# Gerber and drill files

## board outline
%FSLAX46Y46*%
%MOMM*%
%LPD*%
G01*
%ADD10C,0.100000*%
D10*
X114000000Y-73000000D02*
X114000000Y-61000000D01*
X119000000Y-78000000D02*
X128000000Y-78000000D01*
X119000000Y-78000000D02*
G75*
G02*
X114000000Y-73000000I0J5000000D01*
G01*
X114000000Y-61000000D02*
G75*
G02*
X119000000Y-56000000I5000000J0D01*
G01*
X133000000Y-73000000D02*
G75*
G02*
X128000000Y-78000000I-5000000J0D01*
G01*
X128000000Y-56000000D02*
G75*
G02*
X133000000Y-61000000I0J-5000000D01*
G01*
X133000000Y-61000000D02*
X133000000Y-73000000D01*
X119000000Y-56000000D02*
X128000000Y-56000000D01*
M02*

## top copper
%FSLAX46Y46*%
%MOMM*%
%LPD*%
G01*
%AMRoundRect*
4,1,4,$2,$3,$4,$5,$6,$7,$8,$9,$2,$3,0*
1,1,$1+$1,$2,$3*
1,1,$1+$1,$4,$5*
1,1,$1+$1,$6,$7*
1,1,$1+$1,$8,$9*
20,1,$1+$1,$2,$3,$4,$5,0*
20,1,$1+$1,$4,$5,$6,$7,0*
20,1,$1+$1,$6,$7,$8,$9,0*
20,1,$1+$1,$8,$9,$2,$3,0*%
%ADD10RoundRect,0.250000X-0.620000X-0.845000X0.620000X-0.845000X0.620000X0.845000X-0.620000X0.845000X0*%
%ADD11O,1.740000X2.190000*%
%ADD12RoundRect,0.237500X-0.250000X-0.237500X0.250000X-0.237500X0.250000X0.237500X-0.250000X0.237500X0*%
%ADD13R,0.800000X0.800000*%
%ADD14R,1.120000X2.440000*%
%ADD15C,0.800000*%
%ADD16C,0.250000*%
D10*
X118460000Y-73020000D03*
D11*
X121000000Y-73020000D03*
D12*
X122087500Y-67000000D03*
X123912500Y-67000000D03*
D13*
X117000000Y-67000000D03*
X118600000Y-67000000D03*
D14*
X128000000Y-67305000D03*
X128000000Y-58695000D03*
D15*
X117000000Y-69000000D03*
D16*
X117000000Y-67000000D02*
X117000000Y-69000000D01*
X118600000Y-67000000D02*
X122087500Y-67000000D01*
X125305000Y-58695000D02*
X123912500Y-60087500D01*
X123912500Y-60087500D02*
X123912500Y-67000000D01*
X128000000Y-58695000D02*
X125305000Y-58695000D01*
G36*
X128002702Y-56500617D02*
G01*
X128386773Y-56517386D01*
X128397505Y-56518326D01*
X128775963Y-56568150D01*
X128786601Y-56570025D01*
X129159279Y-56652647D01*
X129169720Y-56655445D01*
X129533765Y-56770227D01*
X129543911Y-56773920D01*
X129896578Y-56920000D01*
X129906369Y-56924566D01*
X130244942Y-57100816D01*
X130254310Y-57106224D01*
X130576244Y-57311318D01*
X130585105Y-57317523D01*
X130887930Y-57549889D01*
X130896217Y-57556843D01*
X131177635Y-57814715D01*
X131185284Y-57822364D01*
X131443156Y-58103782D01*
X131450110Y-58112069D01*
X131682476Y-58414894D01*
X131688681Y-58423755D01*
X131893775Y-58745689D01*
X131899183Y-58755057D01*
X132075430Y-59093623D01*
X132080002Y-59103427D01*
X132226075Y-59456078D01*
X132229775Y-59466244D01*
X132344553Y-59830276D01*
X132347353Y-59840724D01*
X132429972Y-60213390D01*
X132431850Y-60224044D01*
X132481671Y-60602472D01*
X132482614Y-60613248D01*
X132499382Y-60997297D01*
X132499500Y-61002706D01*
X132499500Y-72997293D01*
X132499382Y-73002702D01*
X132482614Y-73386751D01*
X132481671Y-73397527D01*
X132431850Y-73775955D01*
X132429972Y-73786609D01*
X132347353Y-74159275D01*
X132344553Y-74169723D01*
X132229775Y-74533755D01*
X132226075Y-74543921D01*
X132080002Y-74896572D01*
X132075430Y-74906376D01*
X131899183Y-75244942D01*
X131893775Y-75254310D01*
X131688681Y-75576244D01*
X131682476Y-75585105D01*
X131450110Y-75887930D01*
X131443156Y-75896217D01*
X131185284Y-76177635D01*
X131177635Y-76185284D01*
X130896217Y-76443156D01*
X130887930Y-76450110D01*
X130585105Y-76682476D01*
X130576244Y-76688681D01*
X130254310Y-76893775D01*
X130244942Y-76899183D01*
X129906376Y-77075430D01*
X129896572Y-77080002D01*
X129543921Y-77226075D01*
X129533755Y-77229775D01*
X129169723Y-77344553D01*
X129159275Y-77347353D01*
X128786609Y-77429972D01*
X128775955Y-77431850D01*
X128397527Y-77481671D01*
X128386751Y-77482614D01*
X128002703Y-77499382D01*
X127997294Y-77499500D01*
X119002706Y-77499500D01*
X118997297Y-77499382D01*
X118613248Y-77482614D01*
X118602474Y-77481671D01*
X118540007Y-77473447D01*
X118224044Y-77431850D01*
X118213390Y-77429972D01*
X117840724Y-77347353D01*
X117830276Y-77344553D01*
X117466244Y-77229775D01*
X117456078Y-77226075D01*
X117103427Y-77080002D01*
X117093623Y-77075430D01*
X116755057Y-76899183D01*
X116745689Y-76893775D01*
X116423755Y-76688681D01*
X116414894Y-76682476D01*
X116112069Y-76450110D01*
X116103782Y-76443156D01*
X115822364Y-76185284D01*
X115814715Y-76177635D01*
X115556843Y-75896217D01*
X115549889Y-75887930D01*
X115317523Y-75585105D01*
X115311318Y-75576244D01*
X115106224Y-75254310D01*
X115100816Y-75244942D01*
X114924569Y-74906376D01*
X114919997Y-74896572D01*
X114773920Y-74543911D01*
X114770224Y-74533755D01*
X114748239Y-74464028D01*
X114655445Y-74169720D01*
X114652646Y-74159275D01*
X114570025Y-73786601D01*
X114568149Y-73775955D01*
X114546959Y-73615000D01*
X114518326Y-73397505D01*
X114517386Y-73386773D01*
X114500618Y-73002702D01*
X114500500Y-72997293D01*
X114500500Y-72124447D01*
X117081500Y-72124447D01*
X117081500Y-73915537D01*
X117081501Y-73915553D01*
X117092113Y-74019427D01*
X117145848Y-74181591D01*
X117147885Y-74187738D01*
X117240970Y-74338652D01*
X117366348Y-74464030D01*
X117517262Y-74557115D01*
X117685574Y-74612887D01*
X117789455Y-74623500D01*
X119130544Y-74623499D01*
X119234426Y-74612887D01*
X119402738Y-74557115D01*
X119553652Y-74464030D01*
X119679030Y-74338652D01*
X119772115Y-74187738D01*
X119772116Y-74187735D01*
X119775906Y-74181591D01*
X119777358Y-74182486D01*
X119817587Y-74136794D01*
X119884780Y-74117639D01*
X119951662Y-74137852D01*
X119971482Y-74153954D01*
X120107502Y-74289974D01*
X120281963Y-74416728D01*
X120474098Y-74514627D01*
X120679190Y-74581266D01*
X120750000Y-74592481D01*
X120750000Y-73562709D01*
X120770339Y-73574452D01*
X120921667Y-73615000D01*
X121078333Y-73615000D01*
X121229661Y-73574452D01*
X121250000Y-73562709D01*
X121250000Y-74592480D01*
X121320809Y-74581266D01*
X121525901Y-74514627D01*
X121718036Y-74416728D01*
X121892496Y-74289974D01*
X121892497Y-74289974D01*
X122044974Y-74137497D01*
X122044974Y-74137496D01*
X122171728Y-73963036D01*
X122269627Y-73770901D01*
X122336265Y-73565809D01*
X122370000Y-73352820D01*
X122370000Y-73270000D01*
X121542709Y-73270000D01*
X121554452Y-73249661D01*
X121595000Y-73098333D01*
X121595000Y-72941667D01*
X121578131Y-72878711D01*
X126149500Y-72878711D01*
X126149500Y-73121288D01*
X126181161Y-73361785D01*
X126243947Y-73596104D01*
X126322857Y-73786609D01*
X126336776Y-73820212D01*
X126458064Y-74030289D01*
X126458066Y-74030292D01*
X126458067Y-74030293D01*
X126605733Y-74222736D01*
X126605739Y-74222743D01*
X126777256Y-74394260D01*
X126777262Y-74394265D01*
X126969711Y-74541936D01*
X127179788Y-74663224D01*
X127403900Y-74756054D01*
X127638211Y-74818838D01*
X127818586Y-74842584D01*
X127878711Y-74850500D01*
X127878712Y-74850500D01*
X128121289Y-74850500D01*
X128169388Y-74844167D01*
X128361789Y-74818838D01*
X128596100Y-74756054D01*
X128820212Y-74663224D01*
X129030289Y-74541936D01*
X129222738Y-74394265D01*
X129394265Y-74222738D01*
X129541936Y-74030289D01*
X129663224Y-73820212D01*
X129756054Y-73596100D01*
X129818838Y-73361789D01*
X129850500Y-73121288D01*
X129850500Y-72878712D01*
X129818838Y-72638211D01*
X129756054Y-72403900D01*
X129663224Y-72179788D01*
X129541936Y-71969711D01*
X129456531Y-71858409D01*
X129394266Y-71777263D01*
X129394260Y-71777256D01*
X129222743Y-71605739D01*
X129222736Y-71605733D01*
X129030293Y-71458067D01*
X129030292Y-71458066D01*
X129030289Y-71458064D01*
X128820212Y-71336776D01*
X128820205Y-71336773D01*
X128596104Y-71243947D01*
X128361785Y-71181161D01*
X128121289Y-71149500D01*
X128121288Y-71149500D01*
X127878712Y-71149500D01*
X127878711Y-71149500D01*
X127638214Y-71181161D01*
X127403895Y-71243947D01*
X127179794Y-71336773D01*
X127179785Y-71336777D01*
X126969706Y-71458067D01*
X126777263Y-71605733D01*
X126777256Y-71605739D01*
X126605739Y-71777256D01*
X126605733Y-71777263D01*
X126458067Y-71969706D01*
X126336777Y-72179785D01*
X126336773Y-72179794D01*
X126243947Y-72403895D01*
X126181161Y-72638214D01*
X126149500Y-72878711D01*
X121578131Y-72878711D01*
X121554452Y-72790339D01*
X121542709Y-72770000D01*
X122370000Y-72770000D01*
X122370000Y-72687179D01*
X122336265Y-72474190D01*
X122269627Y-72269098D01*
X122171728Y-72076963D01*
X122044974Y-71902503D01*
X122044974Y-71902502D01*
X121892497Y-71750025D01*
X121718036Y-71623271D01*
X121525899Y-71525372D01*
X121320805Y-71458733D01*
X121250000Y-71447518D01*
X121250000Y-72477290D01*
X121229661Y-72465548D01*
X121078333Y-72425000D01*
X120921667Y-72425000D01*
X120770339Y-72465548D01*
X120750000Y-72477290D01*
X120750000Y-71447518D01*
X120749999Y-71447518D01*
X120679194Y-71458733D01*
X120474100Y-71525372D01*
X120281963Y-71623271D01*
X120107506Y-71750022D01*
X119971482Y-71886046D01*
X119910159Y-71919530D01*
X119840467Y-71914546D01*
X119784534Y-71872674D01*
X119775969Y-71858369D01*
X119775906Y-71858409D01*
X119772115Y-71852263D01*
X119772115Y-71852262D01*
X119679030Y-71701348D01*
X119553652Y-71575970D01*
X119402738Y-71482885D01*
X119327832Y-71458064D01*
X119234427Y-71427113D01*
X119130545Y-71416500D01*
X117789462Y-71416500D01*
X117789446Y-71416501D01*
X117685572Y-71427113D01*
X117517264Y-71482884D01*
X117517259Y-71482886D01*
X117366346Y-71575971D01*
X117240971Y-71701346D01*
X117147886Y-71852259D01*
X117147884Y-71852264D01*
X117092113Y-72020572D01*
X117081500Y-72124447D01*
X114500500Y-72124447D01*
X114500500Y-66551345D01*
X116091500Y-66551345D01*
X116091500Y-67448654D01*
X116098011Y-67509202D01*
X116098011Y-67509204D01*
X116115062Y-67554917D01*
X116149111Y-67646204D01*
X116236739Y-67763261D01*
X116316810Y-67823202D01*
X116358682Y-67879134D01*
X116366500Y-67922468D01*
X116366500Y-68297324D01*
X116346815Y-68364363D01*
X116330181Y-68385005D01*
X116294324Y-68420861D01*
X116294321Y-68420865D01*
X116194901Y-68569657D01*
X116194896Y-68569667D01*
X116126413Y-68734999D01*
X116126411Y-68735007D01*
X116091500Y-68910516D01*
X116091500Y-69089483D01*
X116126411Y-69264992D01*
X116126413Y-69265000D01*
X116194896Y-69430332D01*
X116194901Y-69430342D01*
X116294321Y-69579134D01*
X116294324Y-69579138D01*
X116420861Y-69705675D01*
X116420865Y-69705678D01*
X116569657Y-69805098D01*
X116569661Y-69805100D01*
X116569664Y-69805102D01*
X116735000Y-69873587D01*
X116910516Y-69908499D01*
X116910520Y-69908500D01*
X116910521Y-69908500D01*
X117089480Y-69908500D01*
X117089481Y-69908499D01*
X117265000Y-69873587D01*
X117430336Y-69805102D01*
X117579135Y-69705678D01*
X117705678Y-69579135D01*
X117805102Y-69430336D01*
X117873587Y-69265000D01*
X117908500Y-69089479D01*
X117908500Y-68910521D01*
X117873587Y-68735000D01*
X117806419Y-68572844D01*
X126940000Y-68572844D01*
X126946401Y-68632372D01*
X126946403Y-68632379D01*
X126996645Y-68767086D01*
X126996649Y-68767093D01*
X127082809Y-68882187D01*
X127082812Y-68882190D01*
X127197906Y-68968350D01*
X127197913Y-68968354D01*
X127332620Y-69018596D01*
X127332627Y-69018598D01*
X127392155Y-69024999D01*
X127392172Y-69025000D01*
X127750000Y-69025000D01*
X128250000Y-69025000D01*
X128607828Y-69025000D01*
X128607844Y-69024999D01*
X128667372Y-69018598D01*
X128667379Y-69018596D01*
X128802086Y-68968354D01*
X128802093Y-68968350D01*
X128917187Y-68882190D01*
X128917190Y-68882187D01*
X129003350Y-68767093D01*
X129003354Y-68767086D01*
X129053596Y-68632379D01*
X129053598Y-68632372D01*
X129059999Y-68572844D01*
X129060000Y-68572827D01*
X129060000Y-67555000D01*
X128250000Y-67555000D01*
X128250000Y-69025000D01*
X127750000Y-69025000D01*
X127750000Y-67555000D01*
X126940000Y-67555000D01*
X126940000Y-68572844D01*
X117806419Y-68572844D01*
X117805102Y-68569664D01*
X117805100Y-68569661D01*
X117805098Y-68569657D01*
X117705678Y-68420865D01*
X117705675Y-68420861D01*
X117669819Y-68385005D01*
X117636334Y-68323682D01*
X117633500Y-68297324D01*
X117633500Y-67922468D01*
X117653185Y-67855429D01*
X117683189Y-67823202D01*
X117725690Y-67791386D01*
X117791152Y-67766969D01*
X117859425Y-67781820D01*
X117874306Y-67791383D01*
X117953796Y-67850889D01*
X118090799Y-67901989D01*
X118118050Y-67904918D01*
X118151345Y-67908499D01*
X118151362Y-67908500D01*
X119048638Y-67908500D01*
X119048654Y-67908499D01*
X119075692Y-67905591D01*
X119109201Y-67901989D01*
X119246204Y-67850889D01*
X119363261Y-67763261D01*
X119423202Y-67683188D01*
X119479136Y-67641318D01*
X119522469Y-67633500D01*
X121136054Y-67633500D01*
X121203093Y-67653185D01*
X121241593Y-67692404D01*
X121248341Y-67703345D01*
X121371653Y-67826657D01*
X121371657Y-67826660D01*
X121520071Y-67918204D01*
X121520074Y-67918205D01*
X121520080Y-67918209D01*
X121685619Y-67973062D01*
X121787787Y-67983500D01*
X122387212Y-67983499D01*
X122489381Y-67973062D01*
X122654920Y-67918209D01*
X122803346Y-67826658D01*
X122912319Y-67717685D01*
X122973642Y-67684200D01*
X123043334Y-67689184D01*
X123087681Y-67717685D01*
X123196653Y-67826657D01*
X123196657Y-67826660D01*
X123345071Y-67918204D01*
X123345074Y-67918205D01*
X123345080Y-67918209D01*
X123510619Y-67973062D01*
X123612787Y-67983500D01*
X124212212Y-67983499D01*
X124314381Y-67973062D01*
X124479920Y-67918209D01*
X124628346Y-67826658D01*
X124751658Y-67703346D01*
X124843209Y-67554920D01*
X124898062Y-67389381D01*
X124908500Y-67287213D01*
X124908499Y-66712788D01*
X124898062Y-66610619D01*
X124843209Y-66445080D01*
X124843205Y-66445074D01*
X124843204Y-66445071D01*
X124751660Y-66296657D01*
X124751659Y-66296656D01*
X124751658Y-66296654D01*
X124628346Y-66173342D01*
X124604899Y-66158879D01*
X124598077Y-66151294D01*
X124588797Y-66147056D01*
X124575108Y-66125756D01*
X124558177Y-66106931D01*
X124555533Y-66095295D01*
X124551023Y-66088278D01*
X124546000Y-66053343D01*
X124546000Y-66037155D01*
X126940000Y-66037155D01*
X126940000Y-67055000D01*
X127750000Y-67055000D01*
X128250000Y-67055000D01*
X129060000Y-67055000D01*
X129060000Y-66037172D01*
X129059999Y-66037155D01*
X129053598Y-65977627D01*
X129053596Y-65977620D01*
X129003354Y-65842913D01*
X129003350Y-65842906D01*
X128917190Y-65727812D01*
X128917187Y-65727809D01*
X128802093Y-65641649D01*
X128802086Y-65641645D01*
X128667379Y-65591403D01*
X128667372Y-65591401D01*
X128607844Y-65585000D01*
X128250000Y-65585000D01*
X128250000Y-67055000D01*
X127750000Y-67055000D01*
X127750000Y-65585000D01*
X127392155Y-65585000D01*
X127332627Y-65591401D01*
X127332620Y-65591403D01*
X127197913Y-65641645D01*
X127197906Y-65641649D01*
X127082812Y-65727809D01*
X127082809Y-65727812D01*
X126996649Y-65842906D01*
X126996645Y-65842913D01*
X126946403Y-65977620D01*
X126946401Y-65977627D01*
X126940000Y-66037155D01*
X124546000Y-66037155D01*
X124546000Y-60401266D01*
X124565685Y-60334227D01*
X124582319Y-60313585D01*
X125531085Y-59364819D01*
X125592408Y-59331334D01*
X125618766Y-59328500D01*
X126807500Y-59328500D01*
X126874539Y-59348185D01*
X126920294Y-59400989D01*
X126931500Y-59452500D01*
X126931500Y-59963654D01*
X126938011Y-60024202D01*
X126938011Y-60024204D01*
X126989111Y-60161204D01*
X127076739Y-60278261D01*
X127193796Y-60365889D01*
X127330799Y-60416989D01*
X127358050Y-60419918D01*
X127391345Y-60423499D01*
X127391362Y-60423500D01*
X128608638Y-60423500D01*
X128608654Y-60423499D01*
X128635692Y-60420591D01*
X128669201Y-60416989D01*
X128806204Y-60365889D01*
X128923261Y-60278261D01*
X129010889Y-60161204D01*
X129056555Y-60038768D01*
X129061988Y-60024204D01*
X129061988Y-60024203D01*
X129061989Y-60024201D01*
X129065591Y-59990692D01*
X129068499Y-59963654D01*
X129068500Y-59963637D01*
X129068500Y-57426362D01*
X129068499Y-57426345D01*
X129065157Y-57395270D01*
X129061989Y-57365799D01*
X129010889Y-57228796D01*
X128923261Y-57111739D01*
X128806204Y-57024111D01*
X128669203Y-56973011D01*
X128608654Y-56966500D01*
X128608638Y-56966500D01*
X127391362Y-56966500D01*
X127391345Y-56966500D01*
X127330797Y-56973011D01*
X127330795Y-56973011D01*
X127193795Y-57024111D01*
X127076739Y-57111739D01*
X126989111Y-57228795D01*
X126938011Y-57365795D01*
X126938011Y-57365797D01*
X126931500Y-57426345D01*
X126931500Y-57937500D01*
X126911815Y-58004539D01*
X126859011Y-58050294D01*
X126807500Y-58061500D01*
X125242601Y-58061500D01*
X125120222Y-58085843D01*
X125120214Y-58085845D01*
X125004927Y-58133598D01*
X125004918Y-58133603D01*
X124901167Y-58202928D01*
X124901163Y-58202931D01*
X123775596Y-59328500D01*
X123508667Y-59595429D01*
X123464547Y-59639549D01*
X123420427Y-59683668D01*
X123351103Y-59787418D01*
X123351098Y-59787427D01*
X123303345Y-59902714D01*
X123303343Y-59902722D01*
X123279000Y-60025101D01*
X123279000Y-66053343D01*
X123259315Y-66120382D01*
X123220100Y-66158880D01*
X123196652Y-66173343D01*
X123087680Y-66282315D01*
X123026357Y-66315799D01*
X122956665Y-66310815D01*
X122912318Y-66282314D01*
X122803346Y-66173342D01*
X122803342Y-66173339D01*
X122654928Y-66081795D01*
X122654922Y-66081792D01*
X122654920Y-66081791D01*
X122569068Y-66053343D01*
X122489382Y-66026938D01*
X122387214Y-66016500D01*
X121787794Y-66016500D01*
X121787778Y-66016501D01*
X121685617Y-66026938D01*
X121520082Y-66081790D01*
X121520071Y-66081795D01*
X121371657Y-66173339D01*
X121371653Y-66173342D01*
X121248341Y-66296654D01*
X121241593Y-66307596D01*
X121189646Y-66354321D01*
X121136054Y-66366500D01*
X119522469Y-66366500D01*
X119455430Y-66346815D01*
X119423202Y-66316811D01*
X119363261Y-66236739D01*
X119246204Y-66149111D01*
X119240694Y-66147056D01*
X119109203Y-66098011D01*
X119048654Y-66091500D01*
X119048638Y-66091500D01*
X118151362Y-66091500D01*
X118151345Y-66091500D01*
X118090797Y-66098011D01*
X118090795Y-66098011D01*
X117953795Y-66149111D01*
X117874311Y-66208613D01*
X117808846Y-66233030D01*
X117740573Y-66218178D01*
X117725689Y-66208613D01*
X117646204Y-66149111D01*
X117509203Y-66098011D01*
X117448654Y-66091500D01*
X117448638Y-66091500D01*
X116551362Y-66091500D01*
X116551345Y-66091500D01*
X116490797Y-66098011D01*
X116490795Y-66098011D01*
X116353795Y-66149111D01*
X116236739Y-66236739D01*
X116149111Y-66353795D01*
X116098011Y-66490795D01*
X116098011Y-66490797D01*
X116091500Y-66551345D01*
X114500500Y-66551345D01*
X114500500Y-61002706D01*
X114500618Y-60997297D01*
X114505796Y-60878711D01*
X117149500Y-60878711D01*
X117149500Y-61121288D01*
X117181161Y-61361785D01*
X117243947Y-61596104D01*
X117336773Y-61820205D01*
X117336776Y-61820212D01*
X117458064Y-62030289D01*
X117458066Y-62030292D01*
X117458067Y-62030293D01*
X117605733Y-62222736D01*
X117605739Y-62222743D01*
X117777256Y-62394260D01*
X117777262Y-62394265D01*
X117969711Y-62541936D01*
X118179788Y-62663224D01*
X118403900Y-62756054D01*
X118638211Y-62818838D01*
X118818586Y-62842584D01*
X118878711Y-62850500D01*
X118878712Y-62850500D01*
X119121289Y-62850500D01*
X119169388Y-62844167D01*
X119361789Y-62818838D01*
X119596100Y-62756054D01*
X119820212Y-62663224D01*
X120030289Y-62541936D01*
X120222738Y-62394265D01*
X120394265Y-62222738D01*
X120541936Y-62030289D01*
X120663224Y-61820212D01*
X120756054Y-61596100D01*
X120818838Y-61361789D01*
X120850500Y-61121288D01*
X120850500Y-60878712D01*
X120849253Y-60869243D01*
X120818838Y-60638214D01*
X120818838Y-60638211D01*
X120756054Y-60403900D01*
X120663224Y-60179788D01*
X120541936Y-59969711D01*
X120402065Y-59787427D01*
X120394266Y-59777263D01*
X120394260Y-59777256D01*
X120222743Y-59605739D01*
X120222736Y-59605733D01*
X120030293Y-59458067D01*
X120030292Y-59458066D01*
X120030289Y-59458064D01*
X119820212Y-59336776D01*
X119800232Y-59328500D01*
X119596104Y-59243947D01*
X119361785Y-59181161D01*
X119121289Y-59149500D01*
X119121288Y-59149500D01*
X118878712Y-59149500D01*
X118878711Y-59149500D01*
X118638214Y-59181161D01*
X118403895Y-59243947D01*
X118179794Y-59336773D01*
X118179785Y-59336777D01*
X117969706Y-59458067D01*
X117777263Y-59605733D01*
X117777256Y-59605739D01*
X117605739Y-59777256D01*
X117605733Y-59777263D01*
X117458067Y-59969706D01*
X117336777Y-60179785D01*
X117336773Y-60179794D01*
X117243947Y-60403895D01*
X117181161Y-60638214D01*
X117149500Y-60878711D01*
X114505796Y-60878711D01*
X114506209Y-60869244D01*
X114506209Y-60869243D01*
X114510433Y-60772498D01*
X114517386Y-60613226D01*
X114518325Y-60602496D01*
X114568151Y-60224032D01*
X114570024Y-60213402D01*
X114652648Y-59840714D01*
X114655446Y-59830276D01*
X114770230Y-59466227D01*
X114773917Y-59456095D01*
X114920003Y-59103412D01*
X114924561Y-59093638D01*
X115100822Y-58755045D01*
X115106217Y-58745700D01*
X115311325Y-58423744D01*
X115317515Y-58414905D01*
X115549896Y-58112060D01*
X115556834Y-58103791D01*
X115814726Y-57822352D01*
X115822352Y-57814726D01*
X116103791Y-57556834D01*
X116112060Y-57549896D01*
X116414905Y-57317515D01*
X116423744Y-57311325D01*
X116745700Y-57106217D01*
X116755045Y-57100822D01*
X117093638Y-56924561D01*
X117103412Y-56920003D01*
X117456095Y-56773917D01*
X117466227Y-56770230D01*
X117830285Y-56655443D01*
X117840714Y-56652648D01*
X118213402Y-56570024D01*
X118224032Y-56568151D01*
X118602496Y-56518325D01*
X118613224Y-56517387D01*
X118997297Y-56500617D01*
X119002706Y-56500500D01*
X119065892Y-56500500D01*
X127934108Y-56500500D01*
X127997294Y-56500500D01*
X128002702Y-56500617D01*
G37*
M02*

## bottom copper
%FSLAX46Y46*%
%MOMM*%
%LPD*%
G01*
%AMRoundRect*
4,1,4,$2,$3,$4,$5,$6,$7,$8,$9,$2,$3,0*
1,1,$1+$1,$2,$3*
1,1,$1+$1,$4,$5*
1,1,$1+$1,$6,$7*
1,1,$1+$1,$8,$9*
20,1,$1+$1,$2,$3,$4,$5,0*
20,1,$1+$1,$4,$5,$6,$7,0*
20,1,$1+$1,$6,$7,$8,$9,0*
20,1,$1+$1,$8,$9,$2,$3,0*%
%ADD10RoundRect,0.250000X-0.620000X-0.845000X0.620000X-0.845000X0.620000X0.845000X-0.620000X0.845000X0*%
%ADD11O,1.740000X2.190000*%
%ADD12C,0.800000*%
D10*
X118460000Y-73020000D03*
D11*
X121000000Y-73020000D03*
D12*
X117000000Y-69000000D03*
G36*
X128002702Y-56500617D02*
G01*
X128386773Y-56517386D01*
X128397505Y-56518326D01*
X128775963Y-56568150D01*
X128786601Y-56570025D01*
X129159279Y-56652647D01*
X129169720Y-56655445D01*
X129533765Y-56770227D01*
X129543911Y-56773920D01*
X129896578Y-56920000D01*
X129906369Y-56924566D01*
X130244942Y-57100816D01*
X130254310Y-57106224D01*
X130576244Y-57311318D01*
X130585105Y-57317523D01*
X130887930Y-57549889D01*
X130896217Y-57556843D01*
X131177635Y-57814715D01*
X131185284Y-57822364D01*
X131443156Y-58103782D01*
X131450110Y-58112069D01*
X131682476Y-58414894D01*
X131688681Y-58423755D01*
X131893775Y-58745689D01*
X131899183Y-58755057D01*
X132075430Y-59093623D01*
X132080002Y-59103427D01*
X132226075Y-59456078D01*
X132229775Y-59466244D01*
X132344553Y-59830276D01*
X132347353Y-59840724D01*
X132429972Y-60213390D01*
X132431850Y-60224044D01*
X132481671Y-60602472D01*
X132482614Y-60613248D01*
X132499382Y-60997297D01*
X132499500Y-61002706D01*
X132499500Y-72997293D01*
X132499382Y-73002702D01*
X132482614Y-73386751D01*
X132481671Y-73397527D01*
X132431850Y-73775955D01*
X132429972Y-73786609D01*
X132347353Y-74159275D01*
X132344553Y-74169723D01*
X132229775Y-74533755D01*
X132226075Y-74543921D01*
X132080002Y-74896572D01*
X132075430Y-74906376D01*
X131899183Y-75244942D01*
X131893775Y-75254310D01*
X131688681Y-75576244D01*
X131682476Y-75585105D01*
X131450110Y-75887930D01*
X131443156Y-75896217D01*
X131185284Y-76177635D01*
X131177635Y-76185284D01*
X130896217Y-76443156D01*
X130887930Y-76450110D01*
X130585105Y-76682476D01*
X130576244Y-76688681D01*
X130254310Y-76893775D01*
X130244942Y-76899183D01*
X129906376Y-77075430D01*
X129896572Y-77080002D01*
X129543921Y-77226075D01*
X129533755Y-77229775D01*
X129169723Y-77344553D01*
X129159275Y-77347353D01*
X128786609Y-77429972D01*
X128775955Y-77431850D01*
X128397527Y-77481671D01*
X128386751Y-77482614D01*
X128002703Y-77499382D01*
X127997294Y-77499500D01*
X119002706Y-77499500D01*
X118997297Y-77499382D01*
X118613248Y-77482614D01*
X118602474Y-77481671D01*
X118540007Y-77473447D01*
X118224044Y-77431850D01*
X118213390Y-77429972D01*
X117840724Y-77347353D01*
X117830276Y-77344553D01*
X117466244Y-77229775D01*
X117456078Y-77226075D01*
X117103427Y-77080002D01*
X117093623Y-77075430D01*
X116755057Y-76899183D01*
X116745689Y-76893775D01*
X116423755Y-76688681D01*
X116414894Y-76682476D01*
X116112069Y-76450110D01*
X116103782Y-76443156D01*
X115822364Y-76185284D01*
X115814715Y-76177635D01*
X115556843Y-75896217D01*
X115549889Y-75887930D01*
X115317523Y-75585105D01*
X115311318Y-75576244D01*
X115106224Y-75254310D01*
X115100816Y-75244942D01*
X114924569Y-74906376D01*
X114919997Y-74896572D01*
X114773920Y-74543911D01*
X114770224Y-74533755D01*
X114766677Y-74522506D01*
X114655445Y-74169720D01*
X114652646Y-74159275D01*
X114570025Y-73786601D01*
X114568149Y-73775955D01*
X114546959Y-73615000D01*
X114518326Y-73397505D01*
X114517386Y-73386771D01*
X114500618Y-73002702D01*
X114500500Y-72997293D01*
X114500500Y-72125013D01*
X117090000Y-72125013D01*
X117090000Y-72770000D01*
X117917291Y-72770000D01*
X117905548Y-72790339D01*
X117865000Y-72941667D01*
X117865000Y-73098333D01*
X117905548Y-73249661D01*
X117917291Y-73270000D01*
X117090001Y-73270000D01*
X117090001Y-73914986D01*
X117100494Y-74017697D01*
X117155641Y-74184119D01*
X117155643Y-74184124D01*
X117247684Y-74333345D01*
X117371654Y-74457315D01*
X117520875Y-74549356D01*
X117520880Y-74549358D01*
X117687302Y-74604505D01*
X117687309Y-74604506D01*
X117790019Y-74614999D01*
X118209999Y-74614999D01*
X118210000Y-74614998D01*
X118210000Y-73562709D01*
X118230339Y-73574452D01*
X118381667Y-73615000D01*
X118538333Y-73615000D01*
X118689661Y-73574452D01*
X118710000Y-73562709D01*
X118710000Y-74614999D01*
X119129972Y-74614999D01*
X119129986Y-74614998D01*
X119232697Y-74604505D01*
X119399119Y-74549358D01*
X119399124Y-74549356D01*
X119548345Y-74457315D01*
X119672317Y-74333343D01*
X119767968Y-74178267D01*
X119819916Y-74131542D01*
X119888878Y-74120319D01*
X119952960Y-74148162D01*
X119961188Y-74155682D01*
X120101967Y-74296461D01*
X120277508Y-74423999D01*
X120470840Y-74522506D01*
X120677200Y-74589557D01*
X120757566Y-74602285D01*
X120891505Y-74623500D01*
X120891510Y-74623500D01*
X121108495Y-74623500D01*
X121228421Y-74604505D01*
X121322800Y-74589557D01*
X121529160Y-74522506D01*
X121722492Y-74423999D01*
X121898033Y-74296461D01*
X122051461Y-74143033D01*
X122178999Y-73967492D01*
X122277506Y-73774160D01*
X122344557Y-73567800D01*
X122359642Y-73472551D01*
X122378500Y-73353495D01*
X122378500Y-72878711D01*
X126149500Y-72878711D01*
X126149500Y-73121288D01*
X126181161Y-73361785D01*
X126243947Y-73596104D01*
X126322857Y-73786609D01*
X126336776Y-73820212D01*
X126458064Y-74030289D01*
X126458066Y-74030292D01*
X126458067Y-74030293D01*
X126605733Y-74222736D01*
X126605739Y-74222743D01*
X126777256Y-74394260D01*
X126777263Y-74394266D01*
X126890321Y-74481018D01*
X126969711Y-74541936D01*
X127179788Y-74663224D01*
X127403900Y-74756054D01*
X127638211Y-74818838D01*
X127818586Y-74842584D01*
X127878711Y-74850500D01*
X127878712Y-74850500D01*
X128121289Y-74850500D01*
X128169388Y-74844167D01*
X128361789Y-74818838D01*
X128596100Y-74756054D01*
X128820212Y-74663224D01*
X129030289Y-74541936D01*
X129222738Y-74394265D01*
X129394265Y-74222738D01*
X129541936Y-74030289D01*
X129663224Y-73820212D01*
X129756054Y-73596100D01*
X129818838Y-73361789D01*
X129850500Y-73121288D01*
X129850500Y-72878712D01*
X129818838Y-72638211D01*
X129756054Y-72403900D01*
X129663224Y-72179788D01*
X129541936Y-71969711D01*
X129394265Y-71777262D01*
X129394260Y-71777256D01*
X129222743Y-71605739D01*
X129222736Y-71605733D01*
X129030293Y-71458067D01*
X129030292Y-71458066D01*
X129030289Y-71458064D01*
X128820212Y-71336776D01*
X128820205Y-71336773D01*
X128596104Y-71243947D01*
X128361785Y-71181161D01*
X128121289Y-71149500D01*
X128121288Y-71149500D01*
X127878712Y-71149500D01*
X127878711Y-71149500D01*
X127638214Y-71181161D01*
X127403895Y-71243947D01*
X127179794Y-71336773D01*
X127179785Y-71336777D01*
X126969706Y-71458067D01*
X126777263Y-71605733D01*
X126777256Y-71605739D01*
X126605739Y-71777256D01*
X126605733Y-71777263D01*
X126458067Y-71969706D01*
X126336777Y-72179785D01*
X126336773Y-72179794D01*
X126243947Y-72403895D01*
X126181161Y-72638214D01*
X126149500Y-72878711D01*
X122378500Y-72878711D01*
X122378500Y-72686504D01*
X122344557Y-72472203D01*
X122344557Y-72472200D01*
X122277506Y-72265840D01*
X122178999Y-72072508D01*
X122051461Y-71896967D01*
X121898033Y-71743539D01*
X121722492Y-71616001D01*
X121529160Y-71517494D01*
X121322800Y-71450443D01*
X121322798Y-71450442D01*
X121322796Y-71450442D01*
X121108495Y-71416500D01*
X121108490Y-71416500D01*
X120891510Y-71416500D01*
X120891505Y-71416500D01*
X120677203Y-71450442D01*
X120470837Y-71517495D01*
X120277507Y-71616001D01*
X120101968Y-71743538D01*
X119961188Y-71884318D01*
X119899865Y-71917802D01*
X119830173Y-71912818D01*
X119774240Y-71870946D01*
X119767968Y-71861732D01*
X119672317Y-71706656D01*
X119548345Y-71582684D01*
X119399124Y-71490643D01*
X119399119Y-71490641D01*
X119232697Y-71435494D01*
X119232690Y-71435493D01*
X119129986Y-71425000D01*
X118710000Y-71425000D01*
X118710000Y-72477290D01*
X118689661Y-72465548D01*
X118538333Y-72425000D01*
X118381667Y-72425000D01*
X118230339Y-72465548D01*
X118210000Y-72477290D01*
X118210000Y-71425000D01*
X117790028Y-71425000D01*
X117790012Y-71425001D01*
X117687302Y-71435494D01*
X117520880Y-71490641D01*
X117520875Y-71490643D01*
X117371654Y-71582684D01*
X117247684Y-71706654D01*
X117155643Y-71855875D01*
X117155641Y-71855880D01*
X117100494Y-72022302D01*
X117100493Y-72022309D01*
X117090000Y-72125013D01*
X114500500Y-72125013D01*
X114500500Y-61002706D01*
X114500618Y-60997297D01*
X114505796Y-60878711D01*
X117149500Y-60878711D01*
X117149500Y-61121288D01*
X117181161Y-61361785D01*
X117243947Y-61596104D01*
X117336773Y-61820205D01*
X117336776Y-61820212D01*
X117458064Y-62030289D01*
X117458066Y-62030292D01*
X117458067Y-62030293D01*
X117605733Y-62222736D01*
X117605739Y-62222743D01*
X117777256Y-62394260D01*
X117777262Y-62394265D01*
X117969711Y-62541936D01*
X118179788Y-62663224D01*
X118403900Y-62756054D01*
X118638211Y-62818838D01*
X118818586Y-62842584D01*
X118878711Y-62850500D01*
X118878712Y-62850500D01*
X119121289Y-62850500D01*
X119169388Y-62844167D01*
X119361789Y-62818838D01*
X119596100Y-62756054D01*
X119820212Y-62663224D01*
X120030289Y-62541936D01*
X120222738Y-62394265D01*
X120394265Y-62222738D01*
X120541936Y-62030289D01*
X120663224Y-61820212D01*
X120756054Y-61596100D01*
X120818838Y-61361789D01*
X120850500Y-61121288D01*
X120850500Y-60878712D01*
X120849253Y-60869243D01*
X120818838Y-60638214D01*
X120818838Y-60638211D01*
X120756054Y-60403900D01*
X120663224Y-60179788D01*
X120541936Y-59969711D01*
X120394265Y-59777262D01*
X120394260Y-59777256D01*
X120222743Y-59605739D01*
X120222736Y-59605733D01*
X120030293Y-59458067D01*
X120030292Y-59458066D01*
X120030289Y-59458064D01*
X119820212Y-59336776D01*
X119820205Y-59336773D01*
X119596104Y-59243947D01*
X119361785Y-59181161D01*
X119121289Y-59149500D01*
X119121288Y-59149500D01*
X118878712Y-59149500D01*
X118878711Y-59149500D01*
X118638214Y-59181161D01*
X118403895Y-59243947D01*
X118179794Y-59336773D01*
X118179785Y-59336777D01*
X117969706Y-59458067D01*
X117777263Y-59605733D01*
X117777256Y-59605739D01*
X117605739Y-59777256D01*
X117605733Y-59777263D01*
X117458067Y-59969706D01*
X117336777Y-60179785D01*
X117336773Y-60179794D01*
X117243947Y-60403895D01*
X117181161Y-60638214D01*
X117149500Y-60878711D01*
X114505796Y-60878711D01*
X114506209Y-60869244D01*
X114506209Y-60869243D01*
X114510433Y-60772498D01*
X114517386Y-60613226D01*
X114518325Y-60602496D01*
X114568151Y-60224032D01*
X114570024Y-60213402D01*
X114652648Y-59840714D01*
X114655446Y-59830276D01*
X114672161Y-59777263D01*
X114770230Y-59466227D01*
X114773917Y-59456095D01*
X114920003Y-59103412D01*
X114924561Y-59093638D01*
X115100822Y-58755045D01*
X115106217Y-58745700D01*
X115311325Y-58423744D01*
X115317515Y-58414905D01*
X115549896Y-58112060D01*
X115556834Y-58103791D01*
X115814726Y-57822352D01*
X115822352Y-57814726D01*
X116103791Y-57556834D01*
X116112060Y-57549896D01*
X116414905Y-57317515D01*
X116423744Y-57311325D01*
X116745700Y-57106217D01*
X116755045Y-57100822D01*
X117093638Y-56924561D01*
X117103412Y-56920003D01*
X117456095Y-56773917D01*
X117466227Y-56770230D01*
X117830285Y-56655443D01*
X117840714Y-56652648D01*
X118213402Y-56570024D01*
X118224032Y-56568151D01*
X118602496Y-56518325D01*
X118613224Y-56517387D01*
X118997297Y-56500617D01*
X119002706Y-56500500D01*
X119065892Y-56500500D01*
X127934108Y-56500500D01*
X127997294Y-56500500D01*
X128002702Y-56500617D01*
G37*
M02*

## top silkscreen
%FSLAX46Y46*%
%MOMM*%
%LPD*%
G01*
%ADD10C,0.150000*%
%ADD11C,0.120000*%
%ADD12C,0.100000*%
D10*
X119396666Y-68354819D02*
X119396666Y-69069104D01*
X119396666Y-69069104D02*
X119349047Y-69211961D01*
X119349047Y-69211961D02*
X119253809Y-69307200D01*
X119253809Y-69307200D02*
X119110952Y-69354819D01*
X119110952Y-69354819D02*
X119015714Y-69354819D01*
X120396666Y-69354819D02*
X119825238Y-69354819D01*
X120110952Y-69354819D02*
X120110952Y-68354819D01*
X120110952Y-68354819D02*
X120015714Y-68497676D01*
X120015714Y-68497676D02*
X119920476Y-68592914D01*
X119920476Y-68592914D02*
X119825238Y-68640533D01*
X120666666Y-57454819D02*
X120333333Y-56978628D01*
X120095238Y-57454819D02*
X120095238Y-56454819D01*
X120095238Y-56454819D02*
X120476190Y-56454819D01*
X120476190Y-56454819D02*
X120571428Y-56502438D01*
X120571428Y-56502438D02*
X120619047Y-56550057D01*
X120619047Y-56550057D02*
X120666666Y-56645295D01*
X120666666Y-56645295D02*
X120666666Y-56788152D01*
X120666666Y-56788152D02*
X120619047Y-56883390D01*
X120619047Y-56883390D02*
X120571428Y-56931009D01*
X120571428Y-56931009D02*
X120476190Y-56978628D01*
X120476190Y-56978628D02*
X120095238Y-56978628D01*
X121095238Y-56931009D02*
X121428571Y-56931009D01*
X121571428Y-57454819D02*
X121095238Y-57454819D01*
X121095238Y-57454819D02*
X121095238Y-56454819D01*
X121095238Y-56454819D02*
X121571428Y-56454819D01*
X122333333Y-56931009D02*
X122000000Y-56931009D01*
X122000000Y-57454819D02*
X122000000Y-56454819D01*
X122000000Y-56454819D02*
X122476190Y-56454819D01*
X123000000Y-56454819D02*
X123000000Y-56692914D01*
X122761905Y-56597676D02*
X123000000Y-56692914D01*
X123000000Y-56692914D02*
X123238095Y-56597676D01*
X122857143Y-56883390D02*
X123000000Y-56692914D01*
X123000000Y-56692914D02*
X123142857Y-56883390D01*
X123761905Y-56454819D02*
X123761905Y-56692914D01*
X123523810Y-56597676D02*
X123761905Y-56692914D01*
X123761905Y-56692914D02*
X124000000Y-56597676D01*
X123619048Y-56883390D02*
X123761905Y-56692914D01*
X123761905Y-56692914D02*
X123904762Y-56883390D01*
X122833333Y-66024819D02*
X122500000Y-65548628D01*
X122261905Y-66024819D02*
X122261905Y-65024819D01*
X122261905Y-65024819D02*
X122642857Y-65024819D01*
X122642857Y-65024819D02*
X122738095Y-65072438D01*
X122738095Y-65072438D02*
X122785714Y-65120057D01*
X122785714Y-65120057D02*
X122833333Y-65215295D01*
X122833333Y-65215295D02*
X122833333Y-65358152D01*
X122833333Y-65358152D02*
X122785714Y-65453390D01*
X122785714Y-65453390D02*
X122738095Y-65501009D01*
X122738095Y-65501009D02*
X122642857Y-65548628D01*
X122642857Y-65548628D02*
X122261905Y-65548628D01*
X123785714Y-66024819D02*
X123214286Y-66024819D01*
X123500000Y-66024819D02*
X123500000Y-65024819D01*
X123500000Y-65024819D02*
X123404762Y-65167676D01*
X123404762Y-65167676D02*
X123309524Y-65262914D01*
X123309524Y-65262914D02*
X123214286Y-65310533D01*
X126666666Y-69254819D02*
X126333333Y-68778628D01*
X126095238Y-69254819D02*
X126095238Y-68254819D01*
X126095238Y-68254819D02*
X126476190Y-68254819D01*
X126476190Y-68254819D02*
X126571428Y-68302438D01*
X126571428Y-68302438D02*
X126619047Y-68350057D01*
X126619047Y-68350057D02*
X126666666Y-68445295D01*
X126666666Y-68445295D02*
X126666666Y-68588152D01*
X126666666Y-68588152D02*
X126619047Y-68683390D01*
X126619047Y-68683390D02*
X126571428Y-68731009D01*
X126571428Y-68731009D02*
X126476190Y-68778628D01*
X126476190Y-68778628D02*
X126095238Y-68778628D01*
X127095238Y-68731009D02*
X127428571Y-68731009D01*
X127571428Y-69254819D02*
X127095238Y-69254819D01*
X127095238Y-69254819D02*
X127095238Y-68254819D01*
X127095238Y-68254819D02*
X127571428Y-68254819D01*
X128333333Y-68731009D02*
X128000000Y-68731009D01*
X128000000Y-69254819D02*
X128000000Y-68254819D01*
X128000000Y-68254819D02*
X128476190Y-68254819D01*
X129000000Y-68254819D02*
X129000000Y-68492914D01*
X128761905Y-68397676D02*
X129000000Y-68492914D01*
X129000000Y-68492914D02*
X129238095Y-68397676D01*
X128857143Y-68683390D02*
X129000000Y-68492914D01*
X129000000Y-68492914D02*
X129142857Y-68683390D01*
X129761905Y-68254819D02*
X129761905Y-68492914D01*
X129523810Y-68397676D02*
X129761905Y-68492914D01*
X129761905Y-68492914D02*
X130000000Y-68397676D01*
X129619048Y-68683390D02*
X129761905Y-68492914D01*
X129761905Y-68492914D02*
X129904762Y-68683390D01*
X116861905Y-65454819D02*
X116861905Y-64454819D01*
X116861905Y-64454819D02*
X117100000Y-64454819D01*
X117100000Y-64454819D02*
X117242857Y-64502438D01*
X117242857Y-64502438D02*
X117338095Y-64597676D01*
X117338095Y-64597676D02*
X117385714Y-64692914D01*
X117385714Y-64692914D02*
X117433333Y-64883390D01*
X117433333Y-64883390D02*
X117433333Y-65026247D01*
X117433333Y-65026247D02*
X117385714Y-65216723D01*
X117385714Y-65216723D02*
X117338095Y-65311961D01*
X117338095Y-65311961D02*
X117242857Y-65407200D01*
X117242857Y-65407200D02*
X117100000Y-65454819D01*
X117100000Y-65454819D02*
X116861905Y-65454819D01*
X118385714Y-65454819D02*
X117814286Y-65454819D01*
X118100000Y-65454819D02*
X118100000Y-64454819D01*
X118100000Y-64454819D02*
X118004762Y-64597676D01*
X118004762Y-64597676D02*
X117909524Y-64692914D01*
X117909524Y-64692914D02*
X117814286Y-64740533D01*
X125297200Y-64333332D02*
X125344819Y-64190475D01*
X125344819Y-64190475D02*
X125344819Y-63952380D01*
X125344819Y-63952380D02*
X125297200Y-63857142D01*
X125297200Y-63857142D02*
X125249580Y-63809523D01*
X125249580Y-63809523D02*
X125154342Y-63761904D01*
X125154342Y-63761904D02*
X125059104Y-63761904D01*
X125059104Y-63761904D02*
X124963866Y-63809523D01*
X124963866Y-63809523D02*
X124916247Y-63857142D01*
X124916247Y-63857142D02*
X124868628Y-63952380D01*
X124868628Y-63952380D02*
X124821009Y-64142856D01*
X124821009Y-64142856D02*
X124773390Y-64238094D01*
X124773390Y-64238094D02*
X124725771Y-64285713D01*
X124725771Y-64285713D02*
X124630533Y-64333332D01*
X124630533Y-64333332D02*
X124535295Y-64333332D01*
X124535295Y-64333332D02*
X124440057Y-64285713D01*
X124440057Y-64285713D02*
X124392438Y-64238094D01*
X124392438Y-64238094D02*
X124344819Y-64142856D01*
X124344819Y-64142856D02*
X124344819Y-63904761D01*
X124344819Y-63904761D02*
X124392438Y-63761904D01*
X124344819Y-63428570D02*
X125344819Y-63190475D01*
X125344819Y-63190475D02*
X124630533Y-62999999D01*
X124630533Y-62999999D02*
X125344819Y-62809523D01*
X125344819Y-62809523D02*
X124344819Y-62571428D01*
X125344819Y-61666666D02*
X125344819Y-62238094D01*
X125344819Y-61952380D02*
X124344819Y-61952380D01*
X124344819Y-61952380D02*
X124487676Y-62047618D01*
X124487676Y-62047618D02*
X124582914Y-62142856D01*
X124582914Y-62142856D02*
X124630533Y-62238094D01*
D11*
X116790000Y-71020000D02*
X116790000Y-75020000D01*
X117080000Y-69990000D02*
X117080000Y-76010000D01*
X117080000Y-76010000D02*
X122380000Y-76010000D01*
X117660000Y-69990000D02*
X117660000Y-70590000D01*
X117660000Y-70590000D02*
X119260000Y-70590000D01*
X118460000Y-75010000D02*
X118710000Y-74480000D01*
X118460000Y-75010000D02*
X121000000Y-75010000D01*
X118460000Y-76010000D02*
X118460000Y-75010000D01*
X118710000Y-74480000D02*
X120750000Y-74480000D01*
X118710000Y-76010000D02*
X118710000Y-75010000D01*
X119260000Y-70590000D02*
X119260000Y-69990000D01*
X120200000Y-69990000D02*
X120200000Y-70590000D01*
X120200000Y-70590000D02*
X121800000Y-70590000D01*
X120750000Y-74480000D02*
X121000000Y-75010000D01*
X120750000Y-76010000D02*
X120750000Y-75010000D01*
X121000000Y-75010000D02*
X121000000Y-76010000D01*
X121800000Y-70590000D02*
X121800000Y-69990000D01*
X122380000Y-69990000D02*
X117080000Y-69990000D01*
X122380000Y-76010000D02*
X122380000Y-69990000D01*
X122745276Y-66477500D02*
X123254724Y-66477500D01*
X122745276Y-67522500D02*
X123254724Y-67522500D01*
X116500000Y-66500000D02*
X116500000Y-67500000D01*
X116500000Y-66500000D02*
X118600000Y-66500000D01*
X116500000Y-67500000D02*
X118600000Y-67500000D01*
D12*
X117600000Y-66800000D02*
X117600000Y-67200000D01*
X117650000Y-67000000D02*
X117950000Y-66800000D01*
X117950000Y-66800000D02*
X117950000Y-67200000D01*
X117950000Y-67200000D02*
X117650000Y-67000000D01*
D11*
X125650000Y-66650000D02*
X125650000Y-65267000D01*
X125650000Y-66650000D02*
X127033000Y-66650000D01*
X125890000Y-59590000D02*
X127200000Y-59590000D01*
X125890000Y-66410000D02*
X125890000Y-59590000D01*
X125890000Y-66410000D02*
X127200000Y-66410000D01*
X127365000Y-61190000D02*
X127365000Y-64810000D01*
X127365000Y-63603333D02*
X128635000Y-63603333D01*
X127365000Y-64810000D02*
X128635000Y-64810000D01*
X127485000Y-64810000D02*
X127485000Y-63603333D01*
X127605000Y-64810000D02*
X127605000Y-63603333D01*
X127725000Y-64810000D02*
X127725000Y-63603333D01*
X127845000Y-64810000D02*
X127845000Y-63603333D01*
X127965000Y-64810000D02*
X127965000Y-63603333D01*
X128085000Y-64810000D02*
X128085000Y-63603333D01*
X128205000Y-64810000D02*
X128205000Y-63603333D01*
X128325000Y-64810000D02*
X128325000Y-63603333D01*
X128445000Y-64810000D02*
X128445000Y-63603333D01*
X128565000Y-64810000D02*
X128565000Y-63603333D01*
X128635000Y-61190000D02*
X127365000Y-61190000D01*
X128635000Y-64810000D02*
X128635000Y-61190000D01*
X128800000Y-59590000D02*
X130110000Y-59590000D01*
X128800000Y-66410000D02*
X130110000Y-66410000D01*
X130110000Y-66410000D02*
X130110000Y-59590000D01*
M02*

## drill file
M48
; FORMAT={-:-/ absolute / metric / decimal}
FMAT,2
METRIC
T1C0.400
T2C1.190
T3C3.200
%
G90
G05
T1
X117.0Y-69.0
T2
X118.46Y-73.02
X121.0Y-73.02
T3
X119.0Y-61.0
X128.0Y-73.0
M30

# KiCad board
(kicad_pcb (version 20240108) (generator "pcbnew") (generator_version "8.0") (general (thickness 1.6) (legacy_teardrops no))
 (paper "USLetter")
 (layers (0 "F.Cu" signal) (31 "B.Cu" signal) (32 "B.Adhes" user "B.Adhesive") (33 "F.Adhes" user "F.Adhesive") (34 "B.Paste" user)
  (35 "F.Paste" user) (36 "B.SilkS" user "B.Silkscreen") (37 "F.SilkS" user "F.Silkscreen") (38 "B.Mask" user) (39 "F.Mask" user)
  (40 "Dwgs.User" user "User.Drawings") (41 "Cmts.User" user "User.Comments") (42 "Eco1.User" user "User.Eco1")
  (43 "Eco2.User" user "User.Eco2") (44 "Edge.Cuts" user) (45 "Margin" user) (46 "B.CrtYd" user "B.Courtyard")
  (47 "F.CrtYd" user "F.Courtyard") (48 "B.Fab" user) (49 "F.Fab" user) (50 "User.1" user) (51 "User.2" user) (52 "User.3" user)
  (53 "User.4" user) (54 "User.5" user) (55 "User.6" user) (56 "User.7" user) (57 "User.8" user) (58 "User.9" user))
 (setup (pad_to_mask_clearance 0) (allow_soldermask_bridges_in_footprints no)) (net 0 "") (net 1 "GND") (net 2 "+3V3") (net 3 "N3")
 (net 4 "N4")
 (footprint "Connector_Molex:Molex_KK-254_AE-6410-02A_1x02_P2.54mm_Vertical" (layer "F.Cu") (at 118.46 73.02)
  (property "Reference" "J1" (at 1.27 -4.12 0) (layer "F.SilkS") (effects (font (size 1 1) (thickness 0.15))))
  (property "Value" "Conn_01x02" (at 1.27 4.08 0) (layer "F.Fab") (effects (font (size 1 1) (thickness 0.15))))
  (fp_line (start -1.67 -2) (end -1.67 2) (stroke (width 0.12) (type solid)) (layer "F.SilkS"))
  (fp_line (start -1.38 -3.03) (end -1.38 2.99) (stroke (width 0.12) (type solid)) (layer "F.SilkS"))
  (fp_line (start -1.38 2.99) (end 3.92 2.99) (stroke (width 0.12) (type solid)) (layer "F.SilkS"))
  (fp_line (start -0.8 -3.03) (end -0.8 -2.43) (stroke (width 0.12) (type solid)) (layer "F.SilkS"))
  (fp_line (start -0.8 -2.43) (end 0.8 -2.43) (stroke (width 0.12) (type solid)) (layer "F.SilkS"))
  (fp_line (start 0 1.99) (end 0.25 1.46) (stroke (width 0.12) (type solid)) (layer "F.SilkS"))
  (fp_line (start 0 1.99) (end 2.54 1.99) (stroke (width 0.12) (type solid)) (layer "F.SilkS"))
  (fp_line (start 0 2.99) (end 0 1.99) (stroke (width 0.12) (type solid)) (layer "F.SilkS"))
  (fp_line (start 0.25 1.46) (end 2.29 1.46) (stroke (width 0.12) (type solid)) (layer "F.SilkS"))
  (fp_line (start 0.25 2.99) (end 0.25 1.99) (stroke (width 0.12) (type solid)) (layer "F.SilkS"))
  (fp_line (start 0.8 -2.43) (end 0.8 -3.03) (stroke (width 0.12) (type solid)) (layer "F.SilkS"))
  (fp_line (start 1.74 -3.03) (end 1.74 -2.43) (stroke (width 0.12) (type solid)) (layer "F.SilkS"))
  (fp_line (start 1.74 -2.43) (end 3.34 -2.43) (stroke (width 0.12) (type solid)) (layer "F.SilkS"))
  (fp_line (start 2.29 1.46) (end 2.54 1.99) (stroke (width 0.12) (type solid)) (layer "F.SilkS"))
  (fp_line (start 2.29 2.99) (end 2.29 1.99) (stroke (width 0.12) (type solid)) (layer "F.SilkS"))
  (fp_line (start 2.54 1.99) (end 2.54 2.99) (stroke (width 0.12) (type solid)) (layer "F.SilkS"))
  (fp_line (start 3.34 -2.43) (end 3.34 -3.03) (stroke (width 0.12) (type solid)) (layer "F.SilkS"))
  (fp_line (start 3.92 -3.03) (end -1.38 -3.03) (stroke (width 0.12) (type solid)) (layer "F.SilkS"))
  (fp_line (start 3.92 2.99) (end 3.92 -3.03) (stroke (width 0.12) (type solid)) (layer "F.SilkS"))
  (pad "1" thru_hole roundrect (at 0 0) (size 1.74 2.19) (drill 1.19) (layers "*.Cu" "*.Mask") (remove_unused_layers no)
   (roundrect_rratio 0.143678) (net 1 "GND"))
  (pad "2" thru_hole oval (at 2.54 0) (size 1.74 2.19) (drill 1.19) (layers "*.Cu" "*.Mask") (remove_unused_layers no) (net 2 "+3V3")))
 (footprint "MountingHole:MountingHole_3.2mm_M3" (layer "F.Cu") (at 119 61)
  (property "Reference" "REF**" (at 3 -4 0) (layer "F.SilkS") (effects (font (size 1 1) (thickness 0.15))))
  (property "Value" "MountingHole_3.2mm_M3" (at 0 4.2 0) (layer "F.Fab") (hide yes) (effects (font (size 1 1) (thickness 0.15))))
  (pad "" np_thru_hole circle (at 0 0) (size 3.2 3.2) (drill 3.2) (layers "*.Cu" "*.Mask")))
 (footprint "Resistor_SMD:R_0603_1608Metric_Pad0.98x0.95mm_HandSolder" (layer "F.Cu") (at 123 67)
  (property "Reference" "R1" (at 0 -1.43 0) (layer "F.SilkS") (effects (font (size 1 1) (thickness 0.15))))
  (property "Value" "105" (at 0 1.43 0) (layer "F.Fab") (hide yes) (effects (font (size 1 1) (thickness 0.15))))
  (fp_line (start -0.254724 -0.5225) (end 0.254724 -0.5225) (stroke (width 0.12) (type solid)) (layer "F.SilkS"))
  (fp_line (start -0.254724 0.5225) (end 0.254724 0.5225) (stroke (width 0.12) (type solid)) (layer "F.SilkS"))
  (pad "1" smd roundrect (at -0.9125 0) (size 0.975 0.95) (layers "F.Cu" "F.Paste" "F.Mask") (roundrect_rratio 0.25) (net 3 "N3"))
  (pad "2" smd roundrect (at 0.9125 0) (size 0.975 0.95) (layers "F.Cu" "F.Paste" "F.Mask") (roundrect_rratio 0.25) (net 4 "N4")))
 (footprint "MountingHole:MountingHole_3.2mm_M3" (layer "F.Cu") (at 128 73)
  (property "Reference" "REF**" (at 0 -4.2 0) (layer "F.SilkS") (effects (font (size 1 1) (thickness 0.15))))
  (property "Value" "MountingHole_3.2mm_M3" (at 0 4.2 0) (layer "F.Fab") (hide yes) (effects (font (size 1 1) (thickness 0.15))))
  (pad "" np_thru_hole circle (at 0 0) (size 3.2 3.2) (drill 3.2) (layers "*.Cu" "*.Mask")))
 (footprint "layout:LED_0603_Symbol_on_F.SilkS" (layer "F.Cu") (at 117.8 67)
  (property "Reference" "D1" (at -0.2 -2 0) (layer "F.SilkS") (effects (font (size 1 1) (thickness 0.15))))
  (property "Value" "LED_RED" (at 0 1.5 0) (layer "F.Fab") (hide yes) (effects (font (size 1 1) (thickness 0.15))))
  (fp_line (start -1.3 -0.5) (end -1.3 0.5) (stroke (width 0.12) (type solid)) (layer "F.SilkS"))
  (fp_line (start -1.3 -0.5) (end 0.8 -0.5) (stroke (width 0.12) (type solid)) (layer "F.SilkS"))
  (fp_line (start -1.3 0.5) (end 0.8 0.5) (stroke (width 0.12) (type solid)) (layer "F.SilkS"))
  (fp_line (start -0.2 -0.2) (end -0.2 0.2) (stroke (width 0.1) (type solid)) (layer "F.SilkS"))
  (fp_line (start -0.15 0) (end 0.15 -0.2) (stroke (width 0.1) (type solid)) (layer "F.SilkS"))
  (fp_line (start 0.15 -0.2) (end 0.15 0.2) (stroke (width 0.1) (type solid)) (layer "F.SilkS"))
  (fp_line (start 0.15 0.2) (end -0.15 0) (stroke (width 0.1) (type solid)) (layer "F.SilkS"))
  (pad "1" smd rect (at -0.8 0 180) (size 0.8 0.8) (layers "F.Cu" "F.Paste" "F.Mask") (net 1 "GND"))
  (pad "2" smd rect (at 0.8 0 180) (size 0.8 0.8) (layers "F.Cu" "F.Paste" "F.Mask") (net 3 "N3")))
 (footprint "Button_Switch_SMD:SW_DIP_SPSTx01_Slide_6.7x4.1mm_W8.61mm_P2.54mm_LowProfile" (layer "F.Cu") (at 128 63 90)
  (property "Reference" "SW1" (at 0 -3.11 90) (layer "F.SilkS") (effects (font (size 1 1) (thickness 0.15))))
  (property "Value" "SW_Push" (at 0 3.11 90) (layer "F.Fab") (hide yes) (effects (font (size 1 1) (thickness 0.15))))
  (fp_line (start -3.65 -2.35) (end -2.267 -2.35) (stroke (width 0.12) (type solid)) (layer "F.SilkS"))
  (fp_line (start -3.65 -2.35) (end -3.65 -0.967) (stroke (width 0.12) (type solid)) (layer "F.SilkS"))
  (fp_line (start 3.41 -2.11) (end 3.41 -0.8) (stroke (width 0.12) (type solid)) (layer "F.SilkS"))
  (fp_line (start -3.41 -2.11) (end 3.41 -2.11) (stroke (width 0.12) (type solid)) (layer "F.SilkS"))
  (fp_line (start -3.41 -2.11) (end -3.41 -0.8) (stroke (width 0.12) (type solid)) (layer "F.SilkS"))
  (fp_line (start 1.81 -0.635) (end -1.81 -0.635) (stroke (width 0.12) (type solid)) (layer "F.SilkS"))
  (fp_line (start -0.603333 -0.635) (end -0.603333 0.635) (stroke (width 0.12) (type solid)) (layer "F.SilkS"))
  (fp_line (start -1.81 -0.635) (end -1.81 0.635) (stroke (width 0.12) (type solid)) (layer "F.SilkS"))
  (fp_line (start -1.81 -0.515) (end -0.603333 -0.515) (stroke (width 0.12) (type solid)) (layer "F.SilkS"))
  (fp_line (start -1.81 -0.395) (end -0.603333 -0.395) (stroke (width 0.12) (type solid)) (layer "F.SilkS"))
  (fp_line (start -1.81 -0.275) (end -0.603333 -0.275) (stroke (width 0.12) (type solid)) (layer "F.SilkS"))
  (fp_line (start -1.81 -0.155) (end -0.603333 -0.155) (stroke (width 0.12) (type solid)) (layer "F.SilkS"))
  (fp_line (start -1.81 -0.035) (end -0.603333 -0.035) (stroke (width 0.12) (type solid)) (layer "F.SilkS"))
  (fp_line (start -1.81 0.085) (end -0.603333 0.085) (stroke (width 0.12) (type solid)) (layer "F.SilkS"))
  (fp_line (start -1.81 0.205) (end -0.603333 0.205) (stroke (width 0.12) (type solid)) (layer "F.SilkS"))
  (fp_line (start -1.81 0.325) (end -0.603333 0.325) (stroke (width 0.12) (type solid)) (layer "F.SilkS"))
  (fp_line (start -1.81 0.445) (end -0.603333 0.445) (stroke (width 0.12) (type solid)) (layer "F.SilkS"))
  (fp_line (start -1.81 0.565) (end -0.603333 0.565) (stroke (width 0.12) (type solid)) (layer "F.SilkS"))
  (fp_line (start 1.81 0.635) (end 1.81 -0.635) (stroke (width 0.12) (type solid)) (layer "F.SilkS"))
  (fp_line (start -1.81 0.635) (end 1.81 0.635) (stroke (width 0.12) (type solid)) (layer "F.SilkS"))
  (fp_line (start 3.41 0.8) (end 3.41 2.11) (stroke (width 0.12) (type solid)) (layer "F.SilkS"))
  (fp_line (start -3.41 0.8) (end -3.41 2.11) (stroke (width 0.12) (type solid)) (layer "F.SilkS"))
  (fp_line (start -3.41 2.11) (end 3.41 2.11) (stroke (width 0.12) (type solid)) (layer "F.SilkS"))
  (pad "1" smd rect (at -4.305 0 90) (size 2.44 1.12) (layers "F.Cu" "F.Paste" "F.Mask") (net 2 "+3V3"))
  (pad "2" smd rect (at 4.305 0 90) (size 2.44 1.12) (layers "F.Cu" "F.Paste" "F.Mask") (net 4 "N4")))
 (gr_line (start 114 73) (end 114 61) (stroke (width 0.1) (type default)) (layer "Edge.Cuts"))
 (gr_line (start 119 78) (end 128 78) (stroke (width 0.1) (type default)) (layer "Edge.Cuts"))
 (gr_arc (start 119 78) (mid 115.464466 76.535534) (end 114 73) (stroke (width 0.1) (type default)) (layer "Edge.Cuts"))
 (gr_arc (start 114 61) (mid 115.464466 57.464466) (end 119 56) (stroke (width 0.1) (type default)) (layer "Edge.Cuts"))
 (gr_arc (start 133 73) (mid 131.535534 76.535534) (end 128 78) (stroke (width 0.1) (type default)) (layer "Edge.Cuts"))
 (gr_arc (start 128 56) (mid 131.535534 57.464466) (end 133 61) (stroke (width 0.1) (type default)) (layer "Edge.Cuts"))
 (gr_line (start 133 61) (end 133 73) (stroke (width 0.1) (type default)) (layer "Edge.Cuts"))
 (gr_line (start 119 56) (end 128 56) (stroke (width 0.1) (type default)) (layer "Edge.Cuts"))
 (segment (start 117 67) (end 117 69) (width 0.25) (layer "F.Cu") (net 1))
 (via (at 117 69) (size 0.8) (drill 0.4) (layers "F.Cu" "B.Cu") (free yes) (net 1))
 (segment (start 118.6 67) (end 122.0875 67) (width 0.25) (layer "F.Cu") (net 3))
 (segment (start 125.305 58.695) (end 123.9125 60.0875) (width 0.25) (layer "F.Cu") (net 4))
 (segment (start 123.9125 60.0875) (end 123.9125 67) (width 0.25) (layer "F.Cu") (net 4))
 (segment (start 128 58.695) (end 125.305 58.695) (width 0.25) (layer "F.Cu") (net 4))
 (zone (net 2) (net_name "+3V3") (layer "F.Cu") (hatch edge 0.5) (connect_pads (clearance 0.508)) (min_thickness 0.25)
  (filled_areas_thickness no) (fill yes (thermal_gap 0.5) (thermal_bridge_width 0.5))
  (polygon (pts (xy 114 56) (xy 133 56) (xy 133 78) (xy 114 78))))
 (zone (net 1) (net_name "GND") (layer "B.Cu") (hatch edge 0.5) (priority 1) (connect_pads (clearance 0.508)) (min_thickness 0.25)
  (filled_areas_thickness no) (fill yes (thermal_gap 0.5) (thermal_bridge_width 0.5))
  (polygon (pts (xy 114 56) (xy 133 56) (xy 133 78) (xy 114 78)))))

